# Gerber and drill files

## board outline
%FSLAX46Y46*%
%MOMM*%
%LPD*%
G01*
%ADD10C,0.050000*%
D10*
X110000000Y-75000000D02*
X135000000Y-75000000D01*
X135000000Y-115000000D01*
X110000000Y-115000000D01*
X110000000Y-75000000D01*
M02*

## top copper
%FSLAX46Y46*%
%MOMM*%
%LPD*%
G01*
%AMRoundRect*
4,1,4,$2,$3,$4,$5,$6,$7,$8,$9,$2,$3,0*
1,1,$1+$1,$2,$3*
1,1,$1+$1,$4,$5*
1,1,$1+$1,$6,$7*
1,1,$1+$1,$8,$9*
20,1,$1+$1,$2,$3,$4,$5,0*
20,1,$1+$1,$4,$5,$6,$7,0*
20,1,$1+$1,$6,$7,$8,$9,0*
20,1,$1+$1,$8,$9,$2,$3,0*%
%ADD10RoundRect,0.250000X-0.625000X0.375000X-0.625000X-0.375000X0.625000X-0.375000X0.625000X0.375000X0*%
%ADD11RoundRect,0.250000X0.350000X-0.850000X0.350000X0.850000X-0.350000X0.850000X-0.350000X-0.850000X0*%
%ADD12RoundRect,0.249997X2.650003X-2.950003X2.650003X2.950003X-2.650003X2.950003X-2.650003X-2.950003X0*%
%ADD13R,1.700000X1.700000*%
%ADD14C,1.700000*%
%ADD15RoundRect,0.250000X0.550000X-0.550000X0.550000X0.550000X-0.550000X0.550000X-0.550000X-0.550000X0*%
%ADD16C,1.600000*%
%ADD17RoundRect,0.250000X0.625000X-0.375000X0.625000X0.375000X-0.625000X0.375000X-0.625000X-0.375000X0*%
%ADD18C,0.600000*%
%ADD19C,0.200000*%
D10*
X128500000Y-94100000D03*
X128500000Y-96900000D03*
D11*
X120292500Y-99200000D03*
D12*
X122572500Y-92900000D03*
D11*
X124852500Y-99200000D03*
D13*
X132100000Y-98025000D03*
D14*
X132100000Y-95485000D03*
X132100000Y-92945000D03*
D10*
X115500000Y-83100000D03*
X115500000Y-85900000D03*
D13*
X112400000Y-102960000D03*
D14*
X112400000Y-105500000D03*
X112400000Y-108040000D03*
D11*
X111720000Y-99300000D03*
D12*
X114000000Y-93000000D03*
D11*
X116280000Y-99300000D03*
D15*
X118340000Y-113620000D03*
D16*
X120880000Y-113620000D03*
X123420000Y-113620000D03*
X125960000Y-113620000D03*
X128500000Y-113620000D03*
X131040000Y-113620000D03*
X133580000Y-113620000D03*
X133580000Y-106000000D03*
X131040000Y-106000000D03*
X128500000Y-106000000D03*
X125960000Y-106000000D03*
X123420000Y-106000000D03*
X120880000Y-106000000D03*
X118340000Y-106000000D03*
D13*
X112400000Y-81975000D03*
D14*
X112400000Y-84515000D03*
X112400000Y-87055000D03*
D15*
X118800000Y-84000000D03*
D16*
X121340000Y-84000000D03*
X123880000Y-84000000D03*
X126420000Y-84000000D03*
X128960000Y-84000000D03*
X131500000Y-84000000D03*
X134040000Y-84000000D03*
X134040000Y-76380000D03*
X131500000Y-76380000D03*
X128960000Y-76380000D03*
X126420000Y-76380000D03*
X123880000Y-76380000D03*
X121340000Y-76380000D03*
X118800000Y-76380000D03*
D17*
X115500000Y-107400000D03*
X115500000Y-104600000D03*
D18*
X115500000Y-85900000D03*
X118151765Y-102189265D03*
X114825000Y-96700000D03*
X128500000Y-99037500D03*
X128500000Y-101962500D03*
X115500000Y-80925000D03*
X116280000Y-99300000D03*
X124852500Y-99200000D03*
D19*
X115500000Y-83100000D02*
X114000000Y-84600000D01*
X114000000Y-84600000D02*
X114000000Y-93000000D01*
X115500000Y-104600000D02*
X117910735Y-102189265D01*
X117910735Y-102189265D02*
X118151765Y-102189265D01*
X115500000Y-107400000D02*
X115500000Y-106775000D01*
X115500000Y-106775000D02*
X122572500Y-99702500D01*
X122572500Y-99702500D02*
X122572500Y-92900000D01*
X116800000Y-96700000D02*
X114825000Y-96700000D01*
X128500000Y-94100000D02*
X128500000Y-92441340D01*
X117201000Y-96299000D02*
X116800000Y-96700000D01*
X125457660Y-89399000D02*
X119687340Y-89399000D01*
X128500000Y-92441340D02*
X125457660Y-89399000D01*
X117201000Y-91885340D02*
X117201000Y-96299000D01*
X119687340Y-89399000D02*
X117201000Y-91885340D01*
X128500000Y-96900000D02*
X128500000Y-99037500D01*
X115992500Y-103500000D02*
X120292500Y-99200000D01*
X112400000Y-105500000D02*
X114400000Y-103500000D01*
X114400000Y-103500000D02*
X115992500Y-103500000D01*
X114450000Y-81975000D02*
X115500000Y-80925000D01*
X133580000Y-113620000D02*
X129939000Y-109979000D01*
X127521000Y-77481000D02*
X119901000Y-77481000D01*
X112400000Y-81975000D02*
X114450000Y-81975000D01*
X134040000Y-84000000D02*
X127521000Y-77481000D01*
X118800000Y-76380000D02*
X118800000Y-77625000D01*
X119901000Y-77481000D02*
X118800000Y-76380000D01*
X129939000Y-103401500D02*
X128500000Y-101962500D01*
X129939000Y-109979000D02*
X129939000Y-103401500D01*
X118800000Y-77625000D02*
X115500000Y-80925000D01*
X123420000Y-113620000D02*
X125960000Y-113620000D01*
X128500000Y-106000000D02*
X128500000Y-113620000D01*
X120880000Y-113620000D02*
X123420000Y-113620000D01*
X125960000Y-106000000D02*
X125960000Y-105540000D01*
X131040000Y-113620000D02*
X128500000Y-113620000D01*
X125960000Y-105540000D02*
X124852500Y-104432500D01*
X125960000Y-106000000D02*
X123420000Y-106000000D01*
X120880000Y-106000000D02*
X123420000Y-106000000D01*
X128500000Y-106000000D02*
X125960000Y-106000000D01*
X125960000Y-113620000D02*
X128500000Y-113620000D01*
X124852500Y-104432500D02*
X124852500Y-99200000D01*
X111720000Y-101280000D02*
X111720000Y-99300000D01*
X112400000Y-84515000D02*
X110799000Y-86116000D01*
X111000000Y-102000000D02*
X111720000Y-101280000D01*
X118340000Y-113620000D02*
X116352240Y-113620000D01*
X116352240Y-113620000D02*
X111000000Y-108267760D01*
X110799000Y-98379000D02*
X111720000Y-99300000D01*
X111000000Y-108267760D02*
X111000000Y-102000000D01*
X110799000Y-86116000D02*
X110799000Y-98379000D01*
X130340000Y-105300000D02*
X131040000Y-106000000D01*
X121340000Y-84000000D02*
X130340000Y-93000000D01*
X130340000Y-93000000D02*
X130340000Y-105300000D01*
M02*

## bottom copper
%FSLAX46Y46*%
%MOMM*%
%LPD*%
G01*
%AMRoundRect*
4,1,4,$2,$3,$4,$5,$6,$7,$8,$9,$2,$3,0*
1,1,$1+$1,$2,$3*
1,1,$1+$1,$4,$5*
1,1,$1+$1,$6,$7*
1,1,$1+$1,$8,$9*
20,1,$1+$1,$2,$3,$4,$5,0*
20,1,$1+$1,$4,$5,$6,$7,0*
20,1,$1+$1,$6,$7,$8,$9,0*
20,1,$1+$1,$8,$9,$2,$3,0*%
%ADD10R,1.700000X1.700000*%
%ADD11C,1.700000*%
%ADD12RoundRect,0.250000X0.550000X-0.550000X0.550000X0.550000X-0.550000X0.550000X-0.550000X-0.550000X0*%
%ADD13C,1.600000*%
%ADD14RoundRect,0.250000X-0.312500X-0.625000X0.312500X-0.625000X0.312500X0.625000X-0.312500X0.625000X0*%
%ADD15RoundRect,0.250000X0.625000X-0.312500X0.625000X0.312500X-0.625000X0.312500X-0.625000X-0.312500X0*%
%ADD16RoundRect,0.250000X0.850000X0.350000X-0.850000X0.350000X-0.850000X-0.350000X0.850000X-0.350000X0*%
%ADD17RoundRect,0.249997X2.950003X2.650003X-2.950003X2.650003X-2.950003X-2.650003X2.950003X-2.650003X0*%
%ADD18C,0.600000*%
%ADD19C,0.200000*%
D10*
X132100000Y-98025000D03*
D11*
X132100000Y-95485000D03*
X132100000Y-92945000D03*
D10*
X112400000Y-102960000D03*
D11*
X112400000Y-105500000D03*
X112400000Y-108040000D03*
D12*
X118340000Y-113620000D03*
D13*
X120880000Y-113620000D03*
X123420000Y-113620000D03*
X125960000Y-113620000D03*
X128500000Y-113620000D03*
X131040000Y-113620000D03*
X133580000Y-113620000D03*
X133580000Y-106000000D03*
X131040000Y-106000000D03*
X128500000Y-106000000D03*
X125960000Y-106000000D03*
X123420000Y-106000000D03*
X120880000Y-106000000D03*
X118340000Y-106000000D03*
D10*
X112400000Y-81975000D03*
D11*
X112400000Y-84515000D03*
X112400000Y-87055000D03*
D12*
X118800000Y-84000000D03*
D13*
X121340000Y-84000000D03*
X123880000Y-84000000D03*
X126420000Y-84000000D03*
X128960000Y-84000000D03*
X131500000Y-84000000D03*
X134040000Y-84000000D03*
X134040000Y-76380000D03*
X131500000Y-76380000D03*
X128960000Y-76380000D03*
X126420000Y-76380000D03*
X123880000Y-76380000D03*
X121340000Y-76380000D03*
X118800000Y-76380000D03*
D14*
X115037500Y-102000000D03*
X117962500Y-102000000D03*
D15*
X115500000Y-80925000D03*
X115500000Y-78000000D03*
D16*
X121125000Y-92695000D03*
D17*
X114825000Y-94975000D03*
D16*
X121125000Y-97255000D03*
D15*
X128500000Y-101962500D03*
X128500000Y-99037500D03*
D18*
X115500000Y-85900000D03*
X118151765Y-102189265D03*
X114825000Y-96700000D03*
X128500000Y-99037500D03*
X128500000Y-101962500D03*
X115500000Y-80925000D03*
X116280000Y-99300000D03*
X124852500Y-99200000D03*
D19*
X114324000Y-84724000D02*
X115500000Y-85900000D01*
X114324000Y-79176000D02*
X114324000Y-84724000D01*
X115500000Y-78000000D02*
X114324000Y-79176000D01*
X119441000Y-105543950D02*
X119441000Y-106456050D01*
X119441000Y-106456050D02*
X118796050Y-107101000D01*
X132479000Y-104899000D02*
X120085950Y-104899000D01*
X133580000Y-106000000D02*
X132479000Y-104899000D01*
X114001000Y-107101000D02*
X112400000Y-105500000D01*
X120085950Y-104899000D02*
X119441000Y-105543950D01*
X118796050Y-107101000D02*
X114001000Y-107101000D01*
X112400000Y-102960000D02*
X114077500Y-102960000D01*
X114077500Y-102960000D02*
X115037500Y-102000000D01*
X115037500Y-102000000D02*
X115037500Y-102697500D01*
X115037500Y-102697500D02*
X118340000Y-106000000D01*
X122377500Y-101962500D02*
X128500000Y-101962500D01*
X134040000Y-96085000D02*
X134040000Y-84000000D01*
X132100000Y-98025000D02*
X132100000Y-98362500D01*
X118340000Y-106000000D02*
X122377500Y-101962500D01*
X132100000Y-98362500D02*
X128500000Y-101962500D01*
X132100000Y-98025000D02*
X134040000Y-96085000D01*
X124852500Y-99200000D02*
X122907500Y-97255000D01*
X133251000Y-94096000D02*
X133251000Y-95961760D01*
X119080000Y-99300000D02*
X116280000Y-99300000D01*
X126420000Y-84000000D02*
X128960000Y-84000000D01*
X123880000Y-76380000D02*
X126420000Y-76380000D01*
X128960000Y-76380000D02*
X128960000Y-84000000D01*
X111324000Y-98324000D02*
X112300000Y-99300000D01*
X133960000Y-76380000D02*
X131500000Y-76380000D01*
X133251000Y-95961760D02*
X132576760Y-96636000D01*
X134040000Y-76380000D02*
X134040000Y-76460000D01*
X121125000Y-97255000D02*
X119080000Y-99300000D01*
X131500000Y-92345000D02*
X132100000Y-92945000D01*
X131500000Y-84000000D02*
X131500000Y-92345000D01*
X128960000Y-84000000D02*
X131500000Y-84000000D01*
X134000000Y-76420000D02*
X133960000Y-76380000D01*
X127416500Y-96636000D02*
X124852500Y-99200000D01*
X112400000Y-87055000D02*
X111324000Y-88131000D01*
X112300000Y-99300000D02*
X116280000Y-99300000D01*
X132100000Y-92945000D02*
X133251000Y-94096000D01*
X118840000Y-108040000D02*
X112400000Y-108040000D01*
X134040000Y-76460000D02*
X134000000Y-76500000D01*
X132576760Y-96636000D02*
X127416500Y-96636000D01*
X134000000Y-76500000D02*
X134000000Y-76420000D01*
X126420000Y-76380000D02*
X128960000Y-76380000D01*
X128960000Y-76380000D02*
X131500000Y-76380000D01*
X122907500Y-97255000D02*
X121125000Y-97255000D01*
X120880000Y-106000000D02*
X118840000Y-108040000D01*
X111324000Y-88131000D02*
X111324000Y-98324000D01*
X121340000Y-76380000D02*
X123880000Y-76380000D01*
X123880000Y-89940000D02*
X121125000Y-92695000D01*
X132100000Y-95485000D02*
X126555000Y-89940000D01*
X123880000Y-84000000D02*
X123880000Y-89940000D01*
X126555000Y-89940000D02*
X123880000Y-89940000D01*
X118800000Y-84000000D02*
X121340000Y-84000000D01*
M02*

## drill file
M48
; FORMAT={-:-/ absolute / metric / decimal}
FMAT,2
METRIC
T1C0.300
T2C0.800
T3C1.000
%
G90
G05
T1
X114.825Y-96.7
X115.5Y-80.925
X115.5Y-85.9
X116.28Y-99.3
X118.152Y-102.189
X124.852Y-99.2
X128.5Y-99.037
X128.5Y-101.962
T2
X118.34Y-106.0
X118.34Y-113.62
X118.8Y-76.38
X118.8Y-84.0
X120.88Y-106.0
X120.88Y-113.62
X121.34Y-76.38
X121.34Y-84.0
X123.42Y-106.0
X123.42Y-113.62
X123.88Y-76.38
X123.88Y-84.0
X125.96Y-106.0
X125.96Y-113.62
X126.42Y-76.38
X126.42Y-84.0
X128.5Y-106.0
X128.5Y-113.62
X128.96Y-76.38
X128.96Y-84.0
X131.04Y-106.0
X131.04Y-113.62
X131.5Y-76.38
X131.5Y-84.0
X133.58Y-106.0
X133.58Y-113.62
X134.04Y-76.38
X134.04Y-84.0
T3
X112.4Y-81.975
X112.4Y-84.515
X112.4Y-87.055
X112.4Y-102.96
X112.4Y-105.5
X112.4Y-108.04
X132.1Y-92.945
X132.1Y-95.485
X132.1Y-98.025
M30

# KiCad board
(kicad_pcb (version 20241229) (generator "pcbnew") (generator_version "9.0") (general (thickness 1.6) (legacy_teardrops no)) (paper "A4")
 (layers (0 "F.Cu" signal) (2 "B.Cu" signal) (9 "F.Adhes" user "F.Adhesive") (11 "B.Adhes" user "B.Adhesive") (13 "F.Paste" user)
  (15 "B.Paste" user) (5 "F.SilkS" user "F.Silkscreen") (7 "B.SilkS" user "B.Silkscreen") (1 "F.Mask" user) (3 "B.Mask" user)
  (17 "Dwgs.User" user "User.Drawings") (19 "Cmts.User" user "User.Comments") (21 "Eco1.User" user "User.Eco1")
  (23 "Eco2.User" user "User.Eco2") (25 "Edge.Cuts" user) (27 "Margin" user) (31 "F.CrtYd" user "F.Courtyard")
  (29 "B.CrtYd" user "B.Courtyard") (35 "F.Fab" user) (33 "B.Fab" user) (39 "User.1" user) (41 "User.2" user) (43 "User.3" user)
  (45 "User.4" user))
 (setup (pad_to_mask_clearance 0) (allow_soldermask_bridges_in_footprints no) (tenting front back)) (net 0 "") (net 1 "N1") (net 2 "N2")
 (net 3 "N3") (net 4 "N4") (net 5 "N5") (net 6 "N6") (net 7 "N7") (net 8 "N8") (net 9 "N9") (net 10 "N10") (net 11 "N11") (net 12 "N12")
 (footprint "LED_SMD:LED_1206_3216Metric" (layer "F.Cu") (at 128.5 95.5 -90)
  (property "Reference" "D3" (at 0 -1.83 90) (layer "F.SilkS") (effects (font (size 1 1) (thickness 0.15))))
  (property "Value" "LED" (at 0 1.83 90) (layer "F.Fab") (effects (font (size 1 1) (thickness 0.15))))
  (pad "1" smd roundrect (at -1.4 0 270) (size 1.25 1.75) (layers "F.Cu" "F.Mask" "F.Paste") (roundrect_rratio 0.2) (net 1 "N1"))
  (pad "2" smd roundrect (at 1.4 0 270) (size 1.25 1.75) (layers "F.Cu" "F.Mask" "F.Paste") (roundrect_rratio 0.2) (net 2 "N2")))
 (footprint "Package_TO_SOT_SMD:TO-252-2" (layer "F.Cu") (at 122.5725 94.16 90)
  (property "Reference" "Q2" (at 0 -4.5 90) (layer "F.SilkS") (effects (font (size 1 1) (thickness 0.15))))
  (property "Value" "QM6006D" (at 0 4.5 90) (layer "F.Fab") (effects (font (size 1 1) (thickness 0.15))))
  (pad "" smd roundrect (at -0.415 -1.525 90) (size 3.05 2.75) (layers "F.Paste") (roundrect_rratio 0.090909))
  (pad "" smd roundrect (at -0.415 1.525 90) (size 3.05 2.75) (layers "F.Paste") (roundrect_rratio 0.090909))
  (pad "" smd roundrect (at 2.935 -1.525 90) (size 3.05 2.75) (layers "F.Paste") (roundrect_rratio 0.090909))
  (pad "" smd roundrect (at 2.935 1.525 90) (size 3.05 2.75) (layers "F.Paste") (roundrect_rratio 0.090909))
  (pad "1" smd roundrect (at -5.04 -2.28 90) (size 2.2 1.2) (layers "F.Cu" "F.Mask" "F.Paste") (roundrect_rratio 0.208333) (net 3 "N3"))
  (pad "2" smd roundrect (at 1.26 0 90) (size 6.4 5.8) (layers "F.Cu" "F.Mask") (roundrect_rratio 0.043103) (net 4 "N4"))
  (pad "3" smd roundrect (at -5.04 2.28 90) (size 2.2 1.2) (layers "F.Cu" "F.Mask" "F.Paste") (roundrect_rratio 0.208333) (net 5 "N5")))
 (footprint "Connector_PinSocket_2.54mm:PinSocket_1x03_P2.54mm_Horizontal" (layer "F.Cu") (at 132.1 98.025 180)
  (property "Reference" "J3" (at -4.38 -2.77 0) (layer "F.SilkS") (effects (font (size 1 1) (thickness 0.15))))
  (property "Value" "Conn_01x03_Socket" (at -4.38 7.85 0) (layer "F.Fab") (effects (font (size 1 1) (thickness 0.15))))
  (pad "1" thru_hole rect (at 0 0 180) (size 1.7 1.7) (drill 1) (layers "*.Cu" "*.Mask") (remove_unused_layers no) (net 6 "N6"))
  (pad "2" thru_hole circle (at 0 2.54 180) (size 1.7 1.7) (drill 1) (layers "*.Cu" "*.Mask") (remove_unused_layers no) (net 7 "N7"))
  (pad "3" thru_hole circle (at 0 5.08 180) (size 1.7 1.7) (drill 1) (layers "*.Cu" "*.Mask") (remove_unused_layers no) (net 5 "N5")))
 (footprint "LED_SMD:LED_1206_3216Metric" (layer "F.Cu") (at 115.5 84.5 -90)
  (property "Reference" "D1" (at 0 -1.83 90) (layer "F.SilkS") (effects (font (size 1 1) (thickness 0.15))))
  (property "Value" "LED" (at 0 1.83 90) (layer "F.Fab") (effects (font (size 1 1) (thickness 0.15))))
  (pad "1" smd roundrect (at -1.4 0 270) (size 1.25 1.75) (layers "F.Cu" "F.Mask" "F.Paste") (roundrect_rratio 0.2) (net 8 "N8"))
  (pad "2" smd roundrect (at 1.4 0 270) (size 1.25 1.75) (layers "F.Cu" "F.Mask" "F.Paste") (roundrect_rratio 0.2) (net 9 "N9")))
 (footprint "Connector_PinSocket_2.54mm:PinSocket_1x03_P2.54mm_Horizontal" (layer "F.Cu") (at 112.4 102.96)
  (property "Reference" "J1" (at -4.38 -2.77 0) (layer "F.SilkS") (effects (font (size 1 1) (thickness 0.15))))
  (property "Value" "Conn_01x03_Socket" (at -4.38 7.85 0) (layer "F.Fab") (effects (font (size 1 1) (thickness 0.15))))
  (pad "1" thru_hole rect (at 0 0) (size 1.7 1.7) (drill 1) (layers "*.Cu" "*.Mask") (remove_unused_layers no) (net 6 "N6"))
  (pad "2" thru_hole circle (at 0 2.54) (size 1.7 1.7) (drill 1) (layers "*.Cu" "*.Mask") (remove_unused_layers no) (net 3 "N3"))
  (pad "3" thru_hole circle (at 0 5.08) (size 1.7 1.7) (drill 1) (layers "*.Cu" "*.Mask") (remove_unused_layers no) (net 5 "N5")))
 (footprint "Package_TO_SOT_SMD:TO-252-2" (layer "F.Cu") (at 114 94.26 90)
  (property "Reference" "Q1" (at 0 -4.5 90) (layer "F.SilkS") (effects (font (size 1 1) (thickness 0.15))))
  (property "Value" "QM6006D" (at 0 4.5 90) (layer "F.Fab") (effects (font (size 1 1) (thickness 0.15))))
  (pad "" smd roundrect (at -0.415 -1.525 90) (size 3.05 2.75) (layers "F.Paste") (roundrect_rratio 0.090909))
  (pad "" smd roundrect (at -0.415 1.525 90) (size 3.05 2.75) (layers "F.Paste") (roundrect_rratio 0.090909))
  (pad "" smd roundrect (at 2.935 -1.525 90) (size 3.05 2.75) (layers "F.Paste") (roundrect_rratio 0.090909))
  (pad "" smd roundrect (at 2.935 1.525 90) (size 3.05 2.75) (layers "F.Paste") (roundrect_rratio 0.090909))
  (pad "1" smd roundrect (at -5.04 -2.28 90) (size 2.2 1.2) (layers "F.Cu" "F.Mask" "F.Paste") (roundrect_rratio 0.208333) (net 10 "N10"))
  (pad "2" smd roundrect (at 1.26 0 90) (size 6.4 5.8) (layers "F.Cu" "F.Mask") (roundrect_rratio 0.043103) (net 8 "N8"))
  (pad "3" smd roundrect (at -5.04 2.28 90) (size 2.2 1.2) (layers "F.Cu" "F.Mask" "F.Paste") (roundrect_rratio 0.208333) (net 5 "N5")))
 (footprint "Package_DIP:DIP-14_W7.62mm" (layer "F.Cu") (at 118.34 113.62 90)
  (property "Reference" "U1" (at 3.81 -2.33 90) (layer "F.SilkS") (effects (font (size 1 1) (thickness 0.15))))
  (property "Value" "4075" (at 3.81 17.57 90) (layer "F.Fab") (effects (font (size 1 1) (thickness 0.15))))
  (pad "1" thru_hole roundrect (at 0 0 90) (size 1.6 1.6) (drill 0.8) (layers "*.Cu" "*.Mask") (remove_unused_layers no)
   (roundrect_rratio 0.15625) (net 10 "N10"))
  (pad "2" thru_hole circle (at 0 2.54 90) (size 1.6 1.6) (drill 0.8) (layers "*.Cu" "*.Mask") (remove_unused_layers no) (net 5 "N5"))
  (pad "3" thru_hole circle (at 0 5.08 90) (size 1.6 1.6) (drill 0.8) (layers "*.Cu" "*.Mask") (remove_unused_layers no) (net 5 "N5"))
  (pad "4" thru_hole circle (at 0 7.62 90) (size 1.6 1.6) (drill 0.8) (layers "*.Cu" "*.Mask") (remove_unused_layers no) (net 5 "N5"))
  (pad "5" thru_hole circle (at 0 10.16 90) (size 1.6 1.6) (drill 0.8) (layers "*.Cu" "*.Mask") (remove_unused_layers no) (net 5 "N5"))
  (pad "6" thru_hole circle (at 0 12.7 90) (size 1.6 1.6) (drill 0.8) (layers "*.Cu" "*.Mask") (remove_unused_layers no) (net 5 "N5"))
  (pad "7" thru_hole circle (at 0 15.24 90) (size 1.6 1.6) (drill 0.8) (layers "*.Cu" "*.Mask") (remove_unused_layers no) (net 6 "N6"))
  (pad "8" thru_hole circle (at 7.62 15.24 90) (size 1.6 1.6) (drill 0.8) (layers "*.Cu" "*.Mask") (remove_unused_layers no) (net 3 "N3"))
  (pad "9" thru_hole circle (at 7.62 12.7 90) (size 1.6 1.6) (drill 0.8) (layers "*.Cu" "*.Mask") (remove_unused_layers no) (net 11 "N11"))
  (pad "10" thru_hole circle (at 7.62 10.16 90) (size 1.6 1.6) (drill 0.8) (layers "*.Cu" "*.Mask") (remove_unused_layers no) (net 5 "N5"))
  (pad "11" thru_hole circle (at 7.62 7.62 90) (size 1.6 1.6) (drill 0.8) (layers "*.Cu" "*.Mask") (remove_unused_layers no) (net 5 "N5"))
  (pad "12" thru_hole circle (at 7.62 5.08 90) (size 1.6 1.6) (drill 0.8) (layers "*.Cu" "*.Mask") (remove_unused_layers no) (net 5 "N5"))
  (pad "13" thru_hole circle (at 7.62 2.54 90) (size 1.6 1.6) (drill 0.8) (layers "*.Cu" "*.Mask") (remove_unused_layers no) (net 5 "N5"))
  (pad "14" thru_hole circle (at 7.62 0 90) (size 1.6 1.6) (drill 0.8) (layers "*.Cu" "*.Mask") (remove_unused_layers no) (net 6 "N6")))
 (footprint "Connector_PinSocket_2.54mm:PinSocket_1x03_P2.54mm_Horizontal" (layer "F.Cu") (at 112.4 81.975)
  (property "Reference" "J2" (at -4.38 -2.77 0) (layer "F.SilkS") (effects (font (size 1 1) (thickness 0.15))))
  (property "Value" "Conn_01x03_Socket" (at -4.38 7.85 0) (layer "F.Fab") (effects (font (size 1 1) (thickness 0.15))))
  (pad "1" thru_hole rect (at 0 0) (size 1.7 1.7) (drill 1) (layers "*.Cu" "*.Mask") (remove_unused_layers no) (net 6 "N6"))
  (pad "2" thru_hole circle (at 0 2.54) (size 1.7 1.7) (drill 1) (layers "*.Cu" "*.Mask") (remove_unused_layers no) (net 10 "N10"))
  (pad "3" thru_hole circle (at 0 5.08) (size 1.7 1.7) (drill 1) (layers "*.Cu" "*.Mask") (remove_unused_layers no) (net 5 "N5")))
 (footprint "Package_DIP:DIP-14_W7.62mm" (layer "F.Cu") (at 118.8 84 90)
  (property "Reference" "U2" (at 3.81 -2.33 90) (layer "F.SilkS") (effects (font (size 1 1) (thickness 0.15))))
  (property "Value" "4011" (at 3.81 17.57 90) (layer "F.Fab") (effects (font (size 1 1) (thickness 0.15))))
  (pad "1" thru_hole roundrect (at 0 0 90) (size 1.6 1.6) (drill 0.8) (layers "*.Cu" "*.Mask") (remove_unused_layers no)
   (roundrect_rratio 0.15625) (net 11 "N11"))
  (pad "2" thru_hole circle (at 0 2.54 90) (size 1.6 1.6) (drill 0.8) (layers "*.Cu" "*.Mask") (remove_unused_layers no) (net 11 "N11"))
  (pad "3" thru_hole circle (at 0 5.08 90) (size 1.6 1.6) (drill 0.8) (layers "*.Cu" "*.Mask") (remove_unused_layers no) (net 7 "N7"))
  (pad "4" thru_hole circle (at 0 7.62 90) (size 1.6 1.6) (drill 0.8) (layers "*.Cu" "*.Mask") (remove_unused_layers no) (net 5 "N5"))
  (pad "5" thru_hole circle (at 0 10.16 90) (size 1.6 1.6) (drill 0.8) (layers "*.Cu" "*.Mask") (remove_unused_layers no) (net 5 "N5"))
  (pad "6" thru_hole circle (at 0 12.7 90) (size 1.6 1.6) (drill 0.8) (layers "*.Cu" "*.Mask") (remove_unused_layers no) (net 5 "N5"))
  (pad "7" thru_hole circle (at 0 15.24 90) (size 1.6 1.6) (drill 0.8) (layers "*.Cu" "*.Mask") (remove_unused_layers no) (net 6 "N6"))
  (pad "8" thru_hole circle (at 7.62 15.24 90) (size 1.6 1.6) (drill 0.8) (layers "*.Cu" "*.Mask") (remove_unused_layers no) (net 5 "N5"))
  (pad "9" thru_hole circle (at 7.62 12.7 90) (size 1.6 1.6) (drill 0.8) (layers "*.Cu" "*.Mask") (remove_unused_layers no) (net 5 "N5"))
  (pad "10" thru_hole circle (at 7.62 10.16 90) (size 1.6 1.6) (drill 0.8) (layers "*.Cu" "*.Mask") (remove_unused_layers no) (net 5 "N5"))
  (pad "11" thru_hole circle (at 7.62 7.62 90) (size 1.6 1.6) (drill 0.8) (layers "*.Cu" "*.Mask") (remove_unused_layers no) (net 5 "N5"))
  (pad "12" thru_hole circle (at 7.62 5.08 90) (size 1.6 1.6) (drill 0.8) (layers "*.Cu" "*.Mask") (remove_unused_layers no) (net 5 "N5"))
  (pad "13" thru_hole circle (at 7.62 2.54 90) (size 1.6 1.6) (drill 0.8) (layers "*.Cu" "*.Mask") (remove_unused_layers no) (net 5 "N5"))
  (pad "14" thru_hole circle (at 7.62 0 90) (size 1.6 1.6) (drill 0.8) (layers "*.Cu" "*.Mask") (remove_unused_layers no) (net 6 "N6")))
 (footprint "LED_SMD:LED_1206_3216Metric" (layer "F.Cu") (at 115.5 106 90)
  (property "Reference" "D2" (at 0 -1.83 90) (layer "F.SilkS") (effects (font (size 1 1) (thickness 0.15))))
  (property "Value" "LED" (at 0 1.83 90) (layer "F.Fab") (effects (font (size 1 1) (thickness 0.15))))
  (pad "1" smd roundrect (at -1.4 0 90) (size 1.25 1.75) (layers "F.Cu" "F.Mask" "F.Paste") (roundrect_rratio 0.2) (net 4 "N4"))
  (pad "2" smd roundrect (at 1.4 0 90) (size 1.25 1.75) (layers "F.Cu" "F.Mask" "F.Paste") (roundrect_rratio 0.2) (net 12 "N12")))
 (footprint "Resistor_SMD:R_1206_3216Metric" (layer "B.Cu") (at 116.5 102)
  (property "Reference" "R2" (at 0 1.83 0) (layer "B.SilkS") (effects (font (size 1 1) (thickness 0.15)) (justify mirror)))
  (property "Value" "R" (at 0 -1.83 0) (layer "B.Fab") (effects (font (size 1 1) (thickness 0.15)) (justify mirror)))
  (pad "1" smd roundrect (at -1.4625 0) (size 1.125 1.75) (layers "B.Cu" "B.Mask" "B.Paste") (roundrect_rratio 0.222222) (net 6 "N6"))
  (pad "2" smd roundrect (at 1.4625 0) (size 1.125 1.75) (layers "B.Cu" "B.Mask" "B.Paste") (roundrect_rratio 0.222222) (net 12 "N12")))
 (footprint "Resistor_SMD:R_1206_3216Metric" (layer "B.Cu") (at 115.5 79.4625 90)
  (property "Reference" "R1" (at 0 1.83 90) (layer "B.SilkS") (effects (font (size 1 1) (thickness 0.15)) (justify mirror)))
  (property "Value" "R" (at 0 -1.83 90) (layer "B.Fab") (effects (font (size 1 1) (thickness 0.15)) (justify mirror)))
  (pad "1" smd roundrect (at -1.4625 0 90) (size 1.125 1.75) (layers "B.Cu" "B.Mask" "B.Paste") (roundrect_rratio 0.222222) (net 6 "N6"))
  (pad "2" smd roundrect (at 1.4625 0 90) (size 1.125 1.75) (layers "B.Cu" "B.Mask" "B.Paste") (roundrect_rratio 0.222222) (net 9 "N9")))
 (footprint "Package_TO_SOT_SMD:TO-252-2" (layer "B.Cu") (at 116.085 94.975 180)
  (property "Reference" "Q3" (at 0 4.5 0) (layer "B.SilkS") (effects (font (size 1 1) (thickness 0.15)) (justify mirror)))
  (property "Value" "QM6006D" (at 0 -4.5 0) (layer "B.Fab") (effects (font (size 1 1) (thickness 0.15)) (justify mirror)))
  (pad "" smd roundrect (at -0.415 -1.525 180) (size 3.05 2.75) (layers "B.Paste") (roundrect_rratio 0.090909))
  (pad "" smd roundrect (at -0.415 1.525 180) (size 3.05 2.75) (layers "B.Paste") (roundrect_rratio 0.090909))
  (pad "" smd roundrect (at 2.935 -1.525 180) (size 3.05 2.75) (layers "B.Paste") (roundrect_rratio 0.090909))
  (pad "" smd roundrect (at 2.935 1.525 180) (size 3.05 2.75) (layers "B.Paste") (roundrect_rratio 0.090909))
  (pad "1" smd roundrect (at -5.04 2.28 180) (size 2.2 1.2) (layers "B.Cu" "B.Mask" "B.Paste") (roundrect_rratio 0.208333) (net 7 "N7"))
  (pad "2" smd roundrect (at 1.26 0 180) (size 6.4 5.8) (layers "B.Cu" "B.Mask") (roundrect_rratio 0.043103) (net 1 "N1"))
  (pad "3" smd roundrect (at -5.04 -2.28 180) (size 2.2 1.2) (layers "B.Cu" "B.Mask" "B.Paste") (roundrect_rratio 0.208333) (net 5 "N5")))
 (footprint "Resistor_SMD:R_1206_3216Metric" (layer "B.Cu") (at 128.5 100.5 90)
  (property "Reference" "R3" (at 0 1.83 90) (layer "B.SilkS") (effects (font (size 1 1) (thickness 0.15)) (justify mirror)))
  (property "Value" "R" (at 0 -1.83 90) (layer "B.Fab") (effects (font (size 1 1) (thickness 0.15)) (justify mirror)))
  (pad "1" smd roundrect (at -1.4625 0 90) (size 1.125 1.75) (layers "B.Cu" "B.Mask" "B.Paste") (roundrect_rratio 0.222222) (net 6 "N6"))
  (pad "2" smd roundrect (at 1.4625 0 90) (size 1.125 1.75) (layers "B.Cu" "B.Mask" "B.Paste") (roundrect_rratio 0.222222) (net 2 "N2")))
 (gr_rect (start 110 75) (end 135 115) (stroke (width 0.05) (type default)) (fill no) (layer "Edge.Cuts"))
 (segment (start 115.5 83.1) (end 114 84.6) (width 0.2) (layer "F.Cu") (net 8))
 (segment (start 114 84.6) (end 114 93) (width 0.2) (layer "F.Cu") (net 8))
 (via (at 115.5 85.9) (size 0.6) (drill 0.3) (layers "F.Cu" "B.Cu") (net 9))
 (segment (start 114.324 84.724) (end 115.5 85.9) (width 0.2) (layer "B.Cu") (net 9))
 (segment (start 114.324 79.176) (end 114.324 84.724) (width 0.2) (layer "B.Cu") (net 9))
 (segment (start 115.5 78) (end 114.324 79.176) (width 0.2) (layer "B.Cu") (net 9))
 (segment (start 115.5 104.6) (end 117.910735 102.189265) (width 0.2) (layer "F.Cu") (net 12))
 (segment (start 117.910735 102.189265) (end 118.151765 102.189265) (width 0.2) (layer "F.Cu") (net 12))
 (via (at 118.151765 102.189265) (size 0.6) (drill 0.3) (layers "F.Cu" "B.Cu") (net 12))
 (segment (start 115.5 107.4) (end 115.5 106.775) (width 0.2) (layer "F.Cu") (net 4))
 (segment (start 115.5 106.775) (end 122.5725 99.7025) (width 0.2) (layer "F.Cu") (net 4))
 (segment (start 122.5725 99.7025) (end 122.5725 92.9) (width 0.2) (layer "F.Cu") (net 4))
 (segment (start 116.8 96.7) (end 114.825 96.7) (width 0.2) (layer "F.Cu") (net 1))
 (segment (start 128.5 94.1) (end 128.5 92.44134) (width 0.2) (layer "F.Cu") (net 1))
 (segment (start 117.201 96.299) (end 116.8 96.7) (width 0.2) (layer "F.Cu") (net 1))
 (segment (start 125.45766 89.399) (end 119.68734 89.399) (width 0.2) (layer "F.Cu") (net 1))
 (segment (start 128.5 92.44134) (end 125.45766 89.399) (width 0.2) (layer "F.Cu") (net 1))
 (segment (start 117.201 91.88534) (end 117.201 96.299) (width 0.2) (layer "F.Cu") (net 1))
 (segment (start 119.68734 89.399) (end 117.201 91.88534) (width 0.2) (layer "F.Cu") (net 1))
 (via (at 114.825 96.7) (size 0.6) (drill 0.3) (layers "F.Cu" "B.Cu") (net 1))
 (segment (start 128.5 96.9) (end 128.5 99.0375) (width 0.2) (layer "F.Cu") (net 2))
 (via (at 128.5 99.0375) (size 0.6) (drill 0.3) (layers "F.Cu" "B.Cu") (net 2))
 (segment (start 115.9925 103.5) (end 120.2925 99.2) (width 0.2) (layer "F.Cu") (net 3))
 (segment (start 112.4 105.5) (end 114.4 103.5) (width 0.2) (layer "F.Cu") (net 3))
 (segment (start 114.4 103.5) (end 115.9925 103.5) (width 0.2) (layer "F.Cu") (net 3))
 (segment (start 119.441 105.54395) (end 119.441 106.45605) (width 0.2) (layer "B.Cu") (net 3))
 (segment (start 119.441 106.45605) (end 118.79605 107.101) (width 0.2) (layer "B.Cu") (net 3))
 (segment (start 132.479 104.899) (end 120.08595 104.899) (width 0.2) (layer "B.Cu") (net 3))
 (segment (start 133.58 106) (end 132.479 104.899) (width 0.2) (layer "B.Cu") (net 3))
 (segment (start 114.001 107.101) (end 112.4 105.5) (width 0.2) (layer "B.Cu") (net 3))
 (segment (start 120.08595 104.899) (end 119.441 105.54395) (width 0.2) (layer "B.Cu") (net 3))
 (segment (start 118.79605 107.101) (end 114.001 107.101) (width 0.2) (layer "B.Cu") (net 3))
 (segment (start 114.45 81.975) (end 115.5 80.925) (width 0.2) (layer "F.Cu") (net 6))
 (segment (start 133.58 113.62) (end 129.939 109.979) (width 0.2) (layer "F.Cu") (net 6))
 (segment (start 127.521 77.481) (end 119.901 77.481) (width 0.2) (layer "F.Cu") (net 6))
 (segment (start 112.4 81.975) (end 114.45 81.975) (width 0.2) (layer "F.Cu") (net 6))
 (segment (start 134.04 84) (end 127.521 77.481) (width 0.2) (layer "F.Cu") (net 6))
 (segment (start 118.8 76.38) (end 118.8 77.625) (width 0.2) (layer "F.Cu") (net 6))
 (segment (start 119.901 77.481) (end 118.8 76.38) (width 0.2) (layer "F.Cu") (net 6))
 (segment (start 129.939 103.4015) (end 128.5 101.9625) (width 0.2) (layer "F.Cu") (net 6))
 (segment (start 129.939 109.979) (end 129.939 103.4015) (width 0.2) (layer "F.Cu") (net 6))
 (segment (start 118.8 77.625) (end 115.5 80.925) (width 0.2) (layer "F.Cu") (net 6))
 (via (at 128.5 101.9625) (size 0.6) (drill 0.3) (layers "F.Cu" "B.Cu") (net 6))
 (via (at 115.5 80.925) (size 0.6) (drill 0.3) (layers "F.Cu" "B.Cu") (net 6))
 (segment (start 112.4 102.96) (end 114.0775 102.96) (width 0.2) (layer "B.Cu") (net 6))
 (segment (start 114.0775 102.96) (end 115.0375 102) (width 0.2) (layer "B.Cu") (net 6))
 (segment (start 115.0375 102) (end 115.0375 102.6975) (width 0.2) (layer "B.Cu") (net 6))
 (segment (start 115.0375 102.6975) (end 118.34 106) (width 0.2) (layer "B.Cu") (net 6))
 (segment (start 122.3775 101.9625) (end 128.5 101.9625) (width 0.2) (layer "B.Cu") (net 6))
 (segment (start 134.04 96.085) (end 134.04 84) (width 0.2) (layer "B.Cu") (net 6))
 (segment (start 132.1 98.025) (end 132.1 98.3625) (width 0.2) (layer "B.Cu") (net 6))
 (segment (start 118.34 106) (end 122.3775 101.9625) (width 0.2) (layer "B.Cu") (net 6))
 (segment (start 132.1 98.3625) (end 128.5 101.9625) (width 0.2) (layer "B.Cu") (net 6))
 (segment (start 132.1 98.025) (end 134.04 96.085) (width 0.2) (layer "B.Cu") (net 6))
 (segment (start 123.42 113.62) (end 125.96 113.62) (width 0.2) (layer "F.Cu") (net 5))
 (segment (start 128.5 106) (end 128.5 113.62) (width 0.2) (layer "F.Cu") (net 5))
 (segment (start 120.88 113.62) (end 123.42 113.62) (width 0.2) (layer "F.Cu") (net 5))
 (segment (start 125.96 106) (end 125.96 105.54) (width 0.2) (layer "F.Cu") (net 5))
 (segment (start 131.04 113.62) (end 128.5 113.62) (width 0.2) (layer "F.Cu") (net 5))
 (segment (start 125.96 105.54) (end 124.8525 104.4325) (width 0.2) (layer "F.Cu") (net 5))
 (segment (start 125.96 106) (end 123.42 106) (width 0.2) (layer "F.Cu") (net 5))
 (segment (start 120.88 106) (end 123.42 106) (width 0.2) (layer "F.Cu") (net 5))
 (segment (start 128.5 106) (end 125.96 106) (width 0.2) (layer "F.Cu") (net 5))
 (segment (start 125.96 113.62) (end 128.5 113.62) (width 0.2) (layer "F.Cu") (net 5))
 (segment (start 124.8525 104.4325) (end 124.8525 99.2) (width 0.2) (layer "F.Cu") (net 5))
 (via (at 116.28 99.3) (size 0.6) (drill 0.3) (layers "F.Cu" "B.Cu") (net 5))
 (via (at 124.8525 99.2) (size 0.6) (drill 0.3) (layers "F.Cu" "B.Cu") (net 5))
 (segment (start 124.8525 99.2) (end 122.9075 97.255) (width 0.2) (layer "B.Cu") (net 5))
 (segment (start 133.251 94.096) (end 133.251 95.96176) (width 0.2) (layer "B.Cu") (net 5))
 (segment (start 119.08 99.3) (end 116.28 99.3) (width 0.2) (layer "B.Cu") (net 5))
 (segment (start 126.42 84) (end 128.96 84) (width 0.2) (layer "B.Cu") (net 5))
 (segment (start 123.88 76.38) (end 126.42 76.38) (width 0.2) (layer "B.Cu") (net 5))
 (segment (start 128.96 76.38) (end 128.96 84) (width 0.2) (layer "B.Cu") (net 5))
 (segment (start 111.324 98.324) (end 112.3 99.3) (width 0.2) (layer "B.Cu") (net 5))
 (segment (start 133.96 76.38) (end 131.5 76.38) (width 0.2) (layer "B.Cu") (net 5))
 (segment (start 133.251 95.96176) (end 132.57676 96.636) (width 0.2) (layer "B.Cu") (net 5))
 (segment (start 134.04 76.38) (end 134.04 76.46) (width 0.2) (layer "B.Cu") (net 5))
 (segment (start 121.125 97.255) (end 119.08 99.3) (width 0.2) (layer "B.Cu") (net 5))
 (segment (start 131.5 92.345) (end 132.1 92.945) (width 0.2) (layer "B.Cu") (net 5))
 (segment (start 131.5 84) (end 131.5 92.345) (width 0.2) (layer "B.Cu") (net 5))
 (segment (start 128.96 84) (end 131.5 84) (width 0.2) (layer "B.Cu") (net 5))
 (segment (start 134 76.42) (end 133.96 76.38) (width 0.2) (layer "B.Cu") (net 5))
 (segment (start 127.4165 96.636) (end 124.8525 99.2) (width 0.2) (layer "B.Cu") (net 5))
 (segment (start 112.4 87.055) (end 111.324 88.131) (width 0.2) (layer "B.Cu") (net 5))
 (segment (start 112.3 99.3) (end 116.28 99.3) (width 0.2) (layer "B.Cu") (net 5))
 (segment (start 132.1 92.945) (end 133.251 94.096) (width 0.2) (layer "B.Cu") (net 5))
 (segment (start 118.84 108.04) (end 112.4 108.04) (width 0.2) (layer "B.Cu") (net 5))
 (segment (start 134.04 76.46) (end 134 76.5) (width 0.2) (layer "B.Cu") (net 5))
 (segment (start 132.57676 96.636) (end 127.4165 96.636) (width 0.2) (layer "B.Cu") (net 5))
 (segment (start 134 76.5) (end 134 76.42) (width 0.2) (layer "B.Cu") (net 5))
 (segment (start 126.42 76.38) (end 128.96 76.38) (width 0.2) (layer "B.Cu") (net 5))
 (segment (start 128.96 76.38) (end 131.5 76.38) (width 0.2) (layer "B.Cu") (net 5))
 (segment (start 122.9075 97.255) (end 121.125 97.255) (width 0.2) (layer "B.Cu") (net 5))
 (segment (start 120.88 106) (end 118.84 108.04) (width 0.2) (layer "B.Cu") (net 5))
 (segment (start 111.324 88.131) (end 111.324 98.324) (width 0.2) (layer "B.Cu") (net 5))
 (segment (start 121.34 76.38) (end 123.88 76.38) (width 0.2) (layer "B.Cu") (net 5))
 (segment (start 111.72 101.28) (end 111.72 99.3) (width 0.2) (layer "F.Cu") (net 10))
 (segment (start 112.4 84.515) (end 110.799 86.116) (width 0.2) (layer "F.Cu") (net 10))
 (segment (start 111 102) (end 111.72 101.28) (width 0.2) (layer "F.Cu") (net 10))
 (segment (start 118.34 113.62) (end 116.35224 113.62) (width 0.2) (layer "F.Cu") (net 10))
 (segment (start 116.35224 113.62) (end 111 108.26776) (width 0.2) (layer "F.Cu") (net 10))
 (segment (start 110.799 98.379) (end 111.72 99.3) (width 0.2) (layer "F.Cu") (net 10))
 (segment (start 111 108.26776) (end 111 102) (width 0.2) (layer "F.Cu") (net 10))
 (segment (start 110.799 86.116) (end 110.799 98.379) (width 0.2) (layer "F.Cu") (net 10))
 (segment (start 123.88 89.94) (end 121.125 92.695) (width 0.2) (layer "B.Cu") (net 7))
 (segment (start 132.1 95.485) (end 126.555 89.94) (width 0.2) (layer "B.Cu") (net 7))
 (segment (start 123.88 84) (end 123.88 89.94) (width 0.2) (layer "B.Cu") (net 7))
 (segment (start 126.555 89.94) (end 123.88 89.94) (width 0.2) (layer "B.Cu") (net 7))
 (segment (start 130.34 105.3) (end 131.04 106) (width 0.2) (layer "F.Cu") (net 11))
 (segment (start 121.34 84) (end 130.34 93) (width 0.2) (layer "F.Cu") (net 11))
 (segment (start 130.34 93) (end 130.34 105.3) (width 0.2) (layer "F.Cu") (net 11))
 (segment (start 118.8 84) (end 121.34 84) (width 0.2) (layer "B.Cu") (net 11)))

